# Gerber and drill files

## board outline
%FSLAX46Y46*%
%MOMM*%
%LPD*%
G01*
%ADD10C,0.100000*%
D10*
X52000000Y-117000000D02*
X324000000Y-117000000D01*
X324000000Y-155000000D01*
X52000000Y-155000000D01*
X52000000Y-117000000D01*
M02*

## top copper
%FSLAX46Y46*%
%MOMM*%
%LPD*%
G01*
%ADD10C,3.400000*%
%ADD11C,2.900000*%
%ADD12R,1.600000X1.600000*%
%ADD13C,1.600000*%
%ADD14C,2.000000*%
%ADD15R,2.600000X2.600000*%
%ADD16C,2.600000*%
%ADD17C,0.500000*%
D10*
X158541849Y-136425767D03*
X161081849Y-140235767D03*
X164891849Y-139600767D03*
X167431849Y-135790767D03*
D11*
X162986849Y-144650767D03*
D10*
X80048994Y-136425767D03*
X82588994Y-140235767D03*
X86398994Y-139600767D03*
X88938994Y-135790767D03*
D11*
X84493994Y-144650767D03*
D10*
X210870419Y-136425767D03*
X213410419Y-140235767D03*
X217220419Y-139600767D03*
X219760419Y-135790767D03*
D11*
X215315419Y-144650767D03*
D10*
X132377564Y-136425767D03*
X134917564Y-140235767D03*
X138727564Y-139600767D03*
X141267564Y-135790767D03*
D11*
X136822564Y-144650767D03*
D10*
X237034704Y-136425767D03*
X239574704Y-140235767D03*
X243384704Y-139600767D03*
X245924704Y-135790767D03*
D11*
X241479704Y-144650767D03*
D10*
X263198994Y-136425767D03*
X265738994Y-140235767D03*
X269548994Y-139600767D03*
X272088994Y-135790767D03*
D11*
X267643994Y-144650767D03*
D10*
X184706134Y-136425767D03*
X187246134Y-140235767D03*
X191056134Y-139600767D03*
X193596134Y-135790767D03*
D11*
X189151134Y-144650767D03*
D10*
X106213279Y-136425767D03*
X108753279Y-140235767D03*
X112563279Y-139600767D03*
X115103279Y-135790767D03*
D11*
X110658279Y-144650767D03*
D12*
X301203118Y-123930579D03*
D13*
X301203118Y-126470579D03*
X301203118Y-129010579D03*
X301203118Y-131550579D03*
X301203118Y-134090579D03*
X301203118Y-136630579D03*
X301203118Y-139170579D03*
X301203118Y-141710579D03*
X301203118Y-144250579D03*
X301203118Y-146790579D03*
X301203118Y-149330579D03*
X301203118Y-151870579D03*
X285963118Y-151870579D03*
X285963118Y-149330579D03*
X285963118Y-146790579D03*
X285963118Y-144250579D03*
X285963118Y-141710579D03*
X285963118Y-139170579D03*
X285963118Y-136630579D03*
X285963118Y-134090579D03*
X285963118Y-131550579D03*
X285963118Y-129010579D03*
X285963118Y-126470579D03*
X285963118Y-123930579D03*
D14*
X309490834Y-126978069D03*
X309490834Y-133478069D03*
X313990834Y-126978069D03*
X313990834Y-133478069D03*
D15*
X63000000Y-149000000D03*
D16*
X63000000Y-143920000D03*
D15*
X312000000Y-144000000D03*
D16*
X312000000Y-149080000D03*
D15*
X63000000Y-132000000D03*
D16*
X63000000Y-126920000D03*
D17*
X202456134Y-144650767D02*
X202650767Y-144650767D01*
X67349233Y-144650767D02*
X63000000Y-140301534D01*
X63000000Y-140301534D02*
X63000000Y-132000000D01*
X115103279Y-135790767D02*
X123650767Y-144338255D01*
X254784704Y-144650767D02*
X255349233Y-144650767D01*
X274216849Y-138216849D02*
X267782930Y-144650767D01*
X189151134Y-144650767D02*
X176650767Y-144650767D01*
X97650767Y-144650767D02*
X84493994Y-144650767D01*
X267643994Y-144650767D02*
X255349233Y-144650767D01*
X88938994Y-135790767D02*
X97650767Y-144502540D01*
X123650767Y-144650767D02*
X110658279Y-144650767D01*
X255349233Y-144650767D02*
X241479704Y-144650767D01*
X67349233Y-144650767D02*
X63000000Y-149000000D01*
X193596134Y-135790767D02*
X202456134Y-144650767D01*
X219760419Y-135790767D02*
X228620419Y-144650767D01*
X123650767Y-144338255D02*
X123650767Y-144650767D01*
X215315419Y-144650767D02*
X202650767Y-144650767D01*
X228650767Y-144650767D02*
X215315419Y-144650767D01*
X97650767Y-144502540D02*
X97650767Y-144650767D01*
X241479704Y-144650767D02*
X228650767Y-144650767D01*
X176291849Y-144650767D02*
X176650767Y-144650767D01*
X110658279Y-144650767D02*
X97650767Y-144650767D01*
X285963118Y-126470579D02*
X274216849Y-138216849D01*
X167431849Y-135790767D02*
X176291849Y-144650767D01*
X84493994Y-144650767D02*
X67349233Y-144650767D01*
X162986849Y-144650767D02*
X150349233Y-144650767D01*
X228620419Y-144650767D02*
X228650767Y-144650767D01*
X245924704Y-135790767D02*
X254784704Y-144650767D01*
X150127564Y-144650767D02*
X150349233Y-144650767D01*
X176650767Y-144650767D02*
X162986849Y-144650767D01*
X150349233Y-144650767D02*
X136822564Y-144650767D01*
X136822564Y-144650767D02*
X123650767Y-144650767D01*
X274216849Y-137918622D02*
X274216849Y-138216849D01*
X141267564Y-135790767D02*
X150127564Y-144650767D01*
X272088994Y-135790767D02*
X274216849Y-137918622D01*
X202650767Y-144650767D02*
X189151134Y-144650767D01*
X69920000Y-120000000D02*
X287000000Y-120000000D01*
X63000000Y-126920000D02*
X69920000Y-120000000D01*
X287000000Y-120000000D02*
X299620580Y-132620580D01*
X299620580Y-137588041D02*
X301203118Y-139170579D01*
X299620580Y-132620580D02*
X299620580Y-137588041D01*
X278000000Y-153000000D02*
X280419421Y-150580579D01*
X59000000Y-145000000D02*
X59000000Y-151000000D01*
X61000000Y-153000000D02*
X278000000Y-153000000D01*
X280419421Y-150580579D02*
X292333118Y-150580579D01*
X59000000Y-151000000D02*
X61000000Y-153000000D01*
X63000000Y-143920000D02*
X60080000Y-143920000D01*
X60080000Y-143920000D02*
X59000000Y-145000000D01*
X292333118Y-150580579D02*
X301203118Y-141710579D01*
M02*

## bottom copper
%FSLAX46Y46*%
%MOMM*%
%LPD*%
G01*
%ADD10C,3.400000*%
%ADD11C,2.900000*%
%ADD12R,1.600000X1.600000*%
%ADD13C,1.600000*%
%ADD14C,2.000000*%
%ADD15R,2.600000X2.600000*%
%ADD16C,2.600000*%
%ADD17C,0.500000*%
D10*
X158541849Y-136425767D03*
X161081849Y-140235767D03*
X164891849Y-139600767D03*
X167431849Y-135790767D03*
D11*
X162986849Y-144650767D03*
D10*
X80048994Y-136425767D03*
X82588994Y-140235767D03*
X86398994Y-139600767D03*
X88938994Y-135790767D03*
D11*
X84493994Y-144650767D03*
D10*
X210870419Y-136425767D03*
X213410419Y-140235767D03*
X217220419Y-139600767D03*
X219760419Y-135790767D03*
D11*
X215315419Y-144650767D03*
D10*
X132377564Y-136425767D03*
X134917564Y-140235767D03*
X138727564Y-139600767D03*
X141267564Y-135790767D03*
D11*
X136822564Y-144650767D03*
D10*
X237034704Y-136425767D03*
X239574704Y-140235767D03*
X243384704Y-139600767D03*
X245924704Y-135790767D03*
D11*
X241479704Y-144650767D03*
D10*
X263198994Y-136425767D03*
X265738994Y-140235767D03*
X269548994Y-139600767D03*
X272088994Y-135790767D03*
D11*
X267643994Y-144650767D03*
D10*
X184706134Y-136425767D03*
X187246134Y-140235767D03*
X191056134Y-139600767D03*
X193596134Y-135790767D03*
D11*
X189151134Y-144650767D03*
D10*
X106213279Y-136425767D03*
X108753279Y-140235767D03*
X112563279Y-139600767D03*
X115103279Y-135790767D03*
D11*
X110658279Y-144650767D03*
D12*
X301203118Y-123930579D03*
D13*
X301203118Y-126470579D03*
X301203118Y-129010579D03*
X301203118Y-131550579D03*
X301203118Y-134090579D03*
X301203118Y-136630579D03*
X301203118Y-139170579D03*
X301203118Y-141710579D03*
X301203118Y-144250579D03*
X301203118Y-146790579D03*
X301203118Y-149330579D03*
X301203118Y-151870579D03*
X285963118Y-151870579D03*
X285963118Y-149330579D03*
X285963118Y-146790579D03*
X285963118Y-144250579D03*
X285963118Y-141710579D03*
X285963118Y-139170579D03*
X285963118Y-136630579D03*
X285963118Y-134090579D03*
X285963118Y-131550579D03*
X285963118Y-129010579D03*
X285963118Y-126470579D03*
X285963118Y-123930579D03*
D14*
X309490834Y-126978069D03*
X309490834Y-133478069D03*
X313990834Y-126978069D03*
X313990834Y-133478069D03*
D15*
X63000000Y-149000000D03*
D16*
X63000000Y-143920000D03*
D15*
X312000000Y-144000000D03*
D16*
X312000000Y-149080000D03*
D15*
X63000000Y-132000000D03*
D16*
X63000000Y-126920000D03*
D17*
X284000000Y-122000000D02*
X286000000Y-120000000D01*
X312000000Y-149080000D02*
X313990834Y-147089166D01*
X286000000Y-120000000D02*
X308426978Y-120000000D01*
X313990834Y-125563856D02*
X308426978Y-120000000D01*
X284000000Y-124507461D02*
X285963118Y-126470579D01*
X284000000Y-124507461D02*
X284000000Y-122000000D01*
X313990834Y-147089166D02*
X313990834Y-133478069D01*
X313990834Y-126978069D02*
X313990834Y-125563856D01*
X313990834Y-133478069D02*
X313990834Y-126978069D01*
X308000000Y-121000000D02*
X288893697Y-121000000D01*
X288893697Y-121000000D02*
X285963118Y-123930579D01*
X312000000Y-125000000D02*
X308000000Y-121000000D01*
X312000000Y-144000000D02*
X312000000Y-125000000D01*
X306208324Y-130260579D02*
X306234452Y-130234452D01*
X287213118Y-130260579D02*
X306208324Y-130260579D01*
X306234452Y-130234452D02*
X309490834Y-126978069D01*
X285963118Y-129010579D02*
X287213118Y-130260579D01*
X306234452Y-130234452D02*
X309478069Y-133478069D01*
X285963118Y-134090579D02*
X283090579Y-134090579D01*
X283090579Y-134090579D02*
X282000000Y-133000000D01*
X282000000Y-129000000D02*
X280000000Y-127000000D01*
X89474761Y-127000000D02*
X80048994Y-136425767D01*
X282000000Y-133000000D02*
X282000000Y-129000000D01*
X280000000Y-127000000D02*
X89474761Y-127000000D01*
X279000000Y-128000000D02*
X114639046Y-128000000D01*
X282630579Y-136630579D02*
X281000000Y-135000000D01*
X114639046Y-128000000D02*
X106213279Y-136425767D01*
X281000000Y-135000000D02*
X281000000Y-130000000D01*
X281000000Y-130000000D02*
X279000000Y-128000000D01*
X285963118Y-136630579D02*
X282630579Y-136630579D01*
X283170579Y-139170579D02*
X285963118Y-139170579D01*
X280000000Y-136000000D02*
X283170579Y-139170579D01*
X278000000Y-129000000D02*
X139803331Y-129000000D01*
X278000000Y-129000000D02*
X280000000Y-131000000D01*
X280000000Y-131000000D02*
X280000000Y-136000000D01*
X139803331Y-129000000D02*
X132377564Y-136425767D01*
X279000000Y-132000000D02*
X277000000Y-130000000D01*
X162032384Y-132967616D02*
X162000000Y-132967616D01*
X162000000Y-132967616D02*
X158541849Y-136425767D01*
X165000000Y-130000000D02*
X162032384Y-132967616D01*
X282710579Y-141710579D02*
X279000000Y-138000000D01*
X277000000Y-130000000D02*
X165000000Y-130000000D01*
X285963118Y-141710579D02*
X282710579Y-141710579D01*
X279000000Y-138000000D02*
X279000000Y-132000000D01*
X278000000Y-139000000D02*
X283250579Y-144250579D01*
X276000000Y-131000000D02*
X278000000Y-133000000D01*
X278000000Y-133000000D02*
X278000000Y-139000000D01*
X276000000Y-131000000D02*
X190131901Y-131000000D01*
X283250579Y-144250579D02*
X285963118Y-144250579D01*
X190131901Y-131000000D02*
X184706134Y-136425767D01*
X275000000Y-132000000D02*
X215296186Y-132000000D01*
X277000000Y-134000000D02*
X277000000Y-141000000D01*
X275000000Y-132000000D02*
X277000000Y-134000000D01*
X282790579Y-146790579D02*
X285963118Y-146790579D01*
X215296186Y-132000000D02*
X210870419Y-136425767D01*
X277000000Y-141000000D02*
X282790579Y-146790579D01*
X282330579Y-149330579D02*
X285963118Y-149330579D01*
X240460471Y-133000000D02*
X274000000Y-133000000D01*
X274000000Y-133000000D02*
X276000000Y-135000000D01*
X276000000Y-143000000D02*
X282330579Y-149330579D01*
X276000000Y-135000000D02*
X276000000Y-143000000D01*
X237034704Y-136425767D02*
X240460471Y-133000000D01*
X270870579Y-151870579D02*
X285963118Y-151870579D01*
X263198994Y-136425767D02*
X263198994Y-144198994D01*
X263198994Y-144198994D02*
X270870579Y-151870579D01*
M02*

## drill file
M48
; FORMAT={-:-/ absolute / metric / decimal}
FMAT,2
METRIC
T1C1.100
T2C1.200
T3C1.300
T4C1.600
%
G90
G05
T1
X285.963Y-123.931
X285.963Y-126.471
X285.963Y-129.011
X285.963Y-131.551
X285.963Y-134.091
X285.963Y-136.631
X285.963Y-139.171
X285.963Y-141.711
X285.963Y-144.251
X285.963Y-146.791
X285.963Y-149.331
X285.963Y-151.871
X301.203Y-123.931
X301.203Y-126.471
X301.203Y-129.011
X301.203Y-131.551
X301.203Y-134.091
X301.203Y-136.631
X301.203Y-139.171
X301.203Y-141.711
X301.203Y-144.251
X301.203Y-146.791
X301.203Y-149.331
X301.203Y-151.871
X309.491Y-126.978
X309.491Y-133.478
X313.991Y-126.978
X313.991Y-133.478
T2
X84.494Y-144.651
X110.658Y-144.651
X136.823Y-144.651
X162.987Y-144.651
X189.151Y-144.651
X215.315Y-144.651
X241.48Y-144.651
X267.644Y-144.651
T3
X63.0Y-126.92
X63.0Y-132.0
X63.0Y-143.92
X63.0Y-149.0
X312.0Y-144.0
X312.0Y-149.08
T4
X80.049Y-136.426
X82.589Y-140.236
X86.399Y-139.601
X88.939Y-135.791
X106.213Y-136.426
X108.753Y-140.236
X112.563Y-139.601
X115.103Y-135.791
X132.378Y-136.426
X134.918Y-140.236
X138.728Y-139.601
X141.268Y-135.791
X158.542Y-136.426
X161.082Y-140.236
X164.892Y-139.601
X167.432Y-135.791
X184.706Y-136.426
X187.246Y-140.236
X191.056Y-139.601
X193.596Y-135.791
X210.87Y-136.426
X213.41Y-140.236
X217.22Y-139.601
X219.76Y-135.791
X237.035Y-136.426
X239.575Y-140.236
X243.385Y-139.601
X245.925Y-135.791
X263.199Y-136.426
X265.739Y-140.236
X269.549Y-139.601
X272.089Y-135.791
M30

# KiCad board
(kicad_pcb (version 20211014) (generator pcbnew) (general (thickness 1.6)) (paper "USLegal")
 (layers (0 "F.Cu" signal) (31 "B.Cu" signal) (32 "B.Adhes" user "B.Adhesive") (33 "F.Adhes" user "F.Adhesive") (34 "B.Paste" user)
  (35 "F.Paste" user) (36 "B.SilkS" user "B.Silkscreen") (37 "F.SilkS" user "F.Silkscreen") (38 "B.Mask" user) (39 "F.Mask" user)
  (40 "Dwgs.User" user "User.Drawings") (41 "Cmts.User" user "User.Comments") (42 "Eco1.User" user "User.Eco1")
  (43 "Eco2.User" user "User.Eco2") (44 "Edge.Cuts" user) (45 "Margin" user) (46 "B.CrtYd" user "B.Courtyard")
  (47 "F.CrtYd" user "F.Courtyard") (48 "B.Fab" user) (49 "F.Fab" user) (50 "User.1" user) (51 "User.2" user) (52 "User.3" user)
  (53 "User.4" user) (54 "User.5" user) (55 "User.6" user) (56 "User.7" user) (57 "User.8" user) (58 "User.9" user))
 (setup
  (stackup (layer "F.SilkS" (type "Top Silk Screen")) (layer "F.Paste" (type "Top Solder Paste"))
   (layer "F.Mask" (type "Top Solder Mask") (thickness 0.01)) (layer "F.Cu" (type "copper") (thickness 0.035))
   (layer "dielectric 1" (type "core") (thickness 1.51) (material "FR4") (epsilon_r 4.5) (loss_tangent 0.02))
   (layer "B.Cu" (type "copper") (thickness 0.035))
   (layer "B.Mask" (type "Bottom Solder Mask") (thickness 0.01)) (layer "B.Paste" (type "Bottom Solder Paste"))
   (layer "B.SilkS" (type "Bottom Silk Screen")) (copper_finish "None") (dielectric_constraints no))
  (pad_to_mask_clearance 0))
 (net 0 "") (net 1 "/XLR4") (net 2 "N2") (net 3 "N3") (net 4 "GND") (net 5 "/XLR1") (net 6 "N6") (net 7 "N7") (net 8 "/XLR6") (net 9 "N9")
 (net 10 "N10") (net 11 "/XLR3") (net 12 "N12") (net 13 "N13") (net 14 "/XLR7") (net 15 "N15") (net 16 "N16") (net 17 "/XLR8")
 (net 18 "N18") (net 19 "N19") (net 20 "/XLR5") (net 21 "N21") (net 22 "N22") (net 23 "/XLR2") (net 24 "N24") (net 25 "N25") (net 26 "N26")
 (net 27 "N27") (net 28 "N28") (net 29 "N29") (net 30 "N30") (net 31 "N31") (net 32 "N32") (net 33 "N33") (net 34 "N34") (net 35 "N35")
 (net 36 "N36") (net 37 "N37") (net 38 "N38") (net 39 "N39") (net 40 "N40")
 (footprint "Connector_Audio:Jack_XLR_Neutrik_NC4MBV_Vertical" (layer "F.Cu") (at 158.541849 136.425767)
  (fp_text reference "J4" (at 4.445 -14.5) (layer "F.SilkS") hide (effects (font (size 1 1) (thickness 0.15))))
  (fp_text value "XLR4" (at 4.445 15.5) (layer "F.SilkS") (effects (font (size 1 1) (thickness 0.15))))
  (pad "1" thru_hole circle (at 0 0) (size 3.4 3.4) (drill 1.6) (layers *.Cu *.Mask) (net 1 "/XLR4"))
  (pad "2" thru_hole circle (at 2.54 3.81) (size 3.4 3.4) (drill 1.6) (layers *.Cu *.Mask) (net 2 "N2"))
  (pad "3" thru_hole circle (at 6.35 3.175) (size 3.4 3.4) (drill 1.6) (layers *.Cu *.Mask) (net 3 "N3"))
  (pad "4" thru_hole circle (at 8.89 -0.635) (size 3.4 3.4) (drill 1.6) (layers *.Cu *.Mask) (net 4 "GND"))
  (pad "G" thru_hole circle (at 4.445 8.225) (size 2.9 2.9) (drill 1.2) (layers *.Cu *.Mask) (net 4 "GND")))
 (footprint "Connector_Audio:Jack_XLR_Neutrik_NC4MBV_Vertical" (layer "F.Cu") (at 80.048994 136.425767)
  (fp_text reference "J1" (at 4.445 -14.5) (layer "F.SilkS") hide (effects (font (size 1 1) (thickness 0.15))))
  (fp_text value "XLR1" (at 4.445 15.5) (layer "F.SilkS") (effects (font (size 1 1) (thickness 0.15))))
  (pad "1" thru_hole circle (at 0 0) (size 3.4 3.4) (drill 1.6) (layers *.Cu *.Mask) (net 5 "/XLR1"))
  (pad "2" thru_hole circle (at 2.54 3.81) (size 3.4 3.4) (drill 1.6) (layers *.Cu *.Mask) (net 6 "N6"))
  (pad "3" thru_hole circle (at 6.35 3.175) (size 3.4 3.4) (drill 1.6) (layers *.Cu *.Mask) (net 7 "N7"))
  (pad "4" thru_hole circle (at 8.89 -0.635) (size 3.4 3.4) (drill 1.6) (layers *.Cu *.Mask) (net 4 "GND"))
  (pad "G" thru_hole circle (at 4.445 8.225) (size 2.9 2.9) (drill 1.2) (layers *.Cu *.Mask) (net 4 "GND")))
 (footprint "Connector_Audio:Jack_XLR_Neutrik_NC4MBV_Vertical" (layer "F.Cu") (at 210.870419 136.425767)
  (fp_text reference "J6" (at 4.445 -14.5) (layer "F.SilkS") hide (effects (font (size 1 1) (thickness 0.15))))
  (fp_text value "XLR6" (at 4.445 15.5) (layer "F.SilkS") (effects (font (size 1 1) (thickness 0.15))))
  (pad "1" thru_hole circle (at 0 0) (size 3.4 3.4) (drill 1.6) (layers *.Cu *.Mask) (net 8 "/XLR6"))
  (pad "2" thru_hole circle (at 2.54 3.81) (size 3.4 3.4) (drill 1.6) (layers *.Cu *.Mask) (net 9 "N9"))
  (pad "3" thru_hole circle (at 6.35 3.175) (size 3.4 3.4) (drill 1.6) (layers *.Cu *.Mask) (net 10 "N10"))
  (pad "4" thru_hole circle (at 8.89 -0.635) (size 3.4 3.4) (drill 1.6) (layers *.Cu *.Mask) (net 4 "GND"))
  (pad "G" thru_hole circle (at 4.445 8.225) (size 2.9 2.9) (drill 1.2) (layers *.Cu *.Mask) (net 4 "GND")))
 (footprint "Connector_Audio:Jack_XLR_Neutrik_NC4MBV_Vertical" (layer "F.Cu") (at 132.377564 136.425767)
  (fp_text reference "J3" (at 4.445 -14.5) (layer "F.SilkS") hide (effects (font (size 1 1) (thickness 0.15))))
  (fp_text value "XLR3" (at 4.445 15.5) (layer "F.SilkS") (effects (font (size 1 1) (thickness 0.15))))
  (pad "1" thru_hole circle (at 0 0) (size 3.4 3.4) (drill 1.6) (layers *.Cu *.Mask) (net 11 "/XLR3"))
  (pad "2" thru_hole circle (at 2.54 3.81) (size 3.4 3.4) (drill 1.6) (layers *.Cu *.Mask) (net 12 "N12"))
  (pad "3" thru_hole circle (at 6.35 3.175) (size 3.4 3.4) (drill 1.6) (layers *.Cu *.Mask) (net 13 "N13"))
  (pad "4" thru_hole circle (at 8.89 -0.635) (size 3.4 3.4) (drill 1.6) (layers *.Cu *.Mask) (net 4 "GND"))
  (pad "G" thru_hole circle (at 4.445 8.225) (size 2.9 2.9) (drill 1.2) (layers *.Cu *.Mask) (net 4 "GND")))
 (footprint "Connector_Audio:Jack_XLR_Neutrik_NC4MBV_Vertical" (layer "F.Cu") (at 237.034704 136.425767)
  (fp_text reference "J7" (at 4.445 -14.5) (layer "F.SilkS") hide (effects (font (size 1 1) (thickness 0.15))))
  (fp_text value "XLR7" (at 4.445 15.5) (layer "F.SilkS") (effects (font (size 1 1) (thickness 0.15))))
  (pad "1" thru_hole circle (at 0 0) (size 3.4 3.4) (drill 1.6) (layers *.Cu *.Mask) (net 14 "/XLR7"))
  (pad "2" thru_hole circle (at 2.54 3.81) (size 3.4 3.4) (drill 1.6) (layers *.Cu *.Mask) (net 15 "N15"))
  (pad "3" thru_hole circle (at 6.35 3.175) (size 3.4 3.4) (drill 1.6) (layers *.Cu *.Mask) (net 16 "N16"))
  (pad "4" thru_hole circle (at 8.89 -0.635) (size 3.4 3.4) (drill 1.6) (layers *.Cu *.Mask) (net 4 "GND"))
  (pad "G" thru_hole circle (at 4.445 8.225) (size 2.9 2.9) (drill 1.2) (layers *.Cu *.Mask) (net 4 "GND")))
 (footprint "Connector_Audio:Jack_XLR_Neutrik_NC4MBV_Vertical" (layer "F.Cu") (at 263.198994 136.425767)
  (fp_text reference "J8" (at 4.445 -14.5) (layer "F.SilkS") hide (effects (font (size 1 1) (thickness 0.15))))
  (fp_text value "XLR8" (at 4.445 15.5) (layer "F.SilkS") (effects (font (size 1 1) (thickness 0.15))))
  (pad "1" thru_hole circle (at 0 0) (size 3.4 3.4) (drill 1.6) (layers *.Cu *.Mask) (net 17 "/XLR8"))
  (pad "2" thru_hole circle (at 2.54 3.81) (size 3.4 3.4) (drill 1.6) (layers *.Cu *.Mask) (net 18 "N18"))
  (pad "3" thru_hole circle (at 6.35 3.175) (size 3.4 3.4) (drill 1.6) (layers *.Cu *.Mask) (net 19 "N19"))
  (pad "4" thru_hole circle (at 8.89 -0.635) (size 3.4 3.4) (drill 1.6) (layers *.Cu *.Mask) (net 4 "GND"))
  (pad "G" thru_hole circle (at 4.445 8.225) (size 2.9 2.9) (drill 1.2) (layers *.Cu *.Mask) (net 4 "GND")))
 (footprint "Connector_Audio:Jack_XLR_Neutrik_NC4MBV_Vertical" (layer "F.Cu") (at 184.706134 136.425767)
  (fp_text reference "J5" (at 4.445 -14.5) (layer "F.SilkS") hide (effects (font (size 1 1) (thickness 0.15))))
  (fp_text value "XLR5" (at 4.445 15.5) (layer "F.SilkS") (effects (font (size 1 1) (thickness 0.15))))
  (pad "1" thru_hole circle (at 0 0) (size 3.4 3.4) (drill 1.6) (layers *.Cu *.Mask) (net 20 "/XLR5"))
  (pad "2" thru_hole circle (at 2.54 3.81) (size 3.4 3.4) (drill 1.6) (layers *.Cu *.Mask) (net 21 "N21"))
  (pad "3" thru_hole circle (at 6.35 3.175) (size 3.4 3.4) (drill 1.6) (layers *.Cu *.Mask) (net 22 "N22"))
  (pad "4" thru_hole circle (at 8.89 -0.635) (size 3.4 3.4) (drill 1.6) (layers *.Cu *.Mask) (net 4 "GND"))
  (pad "G" thru_hole circle (at 4.445 8.225) (size 2.9 2.9) (drill 1.2) (layers *.Cu *.Mask) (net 4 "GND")))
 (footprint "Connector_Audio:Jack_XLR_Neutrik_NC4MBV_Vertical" (layer "F.Cu") (at 106.213279 136.425767)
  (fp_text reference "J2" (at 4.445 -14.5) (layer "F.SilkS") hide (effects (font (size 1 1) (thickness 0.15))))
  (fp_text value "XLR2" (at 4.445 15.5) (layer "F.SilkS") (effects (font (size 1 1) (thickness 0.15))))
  (pad "1" thru_hole circle (at 0 0) (size 3.4 3.4) (drill 1.6) (layers *.Cu *.Mask) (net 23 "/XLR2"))
  (pad "2" thru_hole circle (at 2.54 3.81) (size 3.4 3.4) (drill 1.6) (layers *.Cu *.Mask) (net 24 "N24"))
  (pad "3" thru_hole circle (at 6.35 3.175) (size 3.4 3.4) (drill 1.6) (layers *.Cu *.Mask) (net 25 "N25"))
  (pad "4" thru_hole circle (at 8.89 -0.635) (size 3.4 3.4) (drill 1.6) (layers *.Cu *.Mask) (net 4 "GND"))
  (pad "G" thru_hole circle (at 4.445 8.225) (size 2.9 2.9) (drill 1.2) (layers *.Cu *.Mask) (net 4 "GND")))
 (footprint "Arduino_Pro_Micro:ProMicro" (layer "B.Cu") (at 293.583118 137.900579 -90)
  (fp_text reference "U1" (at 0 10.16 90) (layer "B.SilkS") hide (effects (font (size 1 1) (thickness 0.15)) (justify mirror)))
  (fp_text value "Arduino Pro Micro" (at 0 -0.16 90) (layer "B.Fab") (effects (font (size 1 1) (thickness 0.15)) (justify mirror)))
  (pad "1" thru_hole rect locked (at -13.97 -7.62 270) (size 1.6 1.6) (drill 1.1) (layers *.Cu *.Mask "B.SilkS") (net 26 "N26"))
  (pad "2" thru_hole circle locked (at -11.43 -7.62 270) (size 1.6 1.6) (drill 1.1) (layers *.Cu *.Mask "B.SilkS") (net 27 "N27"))
  (pad "3" thru_hole circle locked (at -8.89 -7.62 270) (size 1.6 1.6) (drill 1.1) (layers *.Cu *.Mask "B.SilkS") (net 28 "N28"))
  (pad "4" thru_hole circle locked (at -6.35 -7.62 270) (size 1.6 1.6) (drill 1.1) (layers *.Cu *.Mask "B.SilkS") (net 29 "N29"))
  (pad "5" thru_hole circle locked (at -3.81 -7.62 270) (size 1.6 1.6) (drill 1.1) (layers *.Cu *.Mask "B.SilkS") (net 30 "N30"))
  (pad "6" thru_hole circle locked (at -1.27 -7.62 270) (size 1.6 1.6) (drill 1.1) (layers *.Cu *.Mask "B.SilkS") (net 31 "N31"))
  (pad "7" thru_hole circle locked (at 1.27 -7.62 270) (size 1.6 1.6) (drill 1.1) (layers *.Cu *.Mask "B.SilkS") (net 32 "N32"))
  (pad "8" thru_hole circle locked (at 3.81 -7.62 270) (size 1.6 1.6) (drill 1.1) (layers *.Cu *.Mask "B.SilkS") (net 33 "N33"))
  (pad "9" thru_hole circle locked (at 6.35 -7.62 270) (size 1.6 1.6) (drill 1.1) (layers *.Cu *.Mask "B.SilkS") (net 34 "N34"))
  (pad "10" thru_hole circle locked (at 8.89 -7.62 270) (size 1.6 1.6) (drill 1.1) (layers *.Cu *.Mask "B.SilkS") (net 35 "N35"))
  (pad "11" thru_hole circle locked (at 11.43 -7.62 270) (size 1.6 1.6) (drill 1.1) (layers *.Cu *.Mask "B.SilkS") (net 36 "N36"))
  (pad "12" thru_hole circle locked (at 13.97 -7.62 270) (size 1.6 1.6) (drill 1.1) (layers *.Cu *.Mask "B.SilkS") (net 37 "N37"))
  (pad "13" thru_hole circle locked (at 13.97 7.62 270) (size 1.6 1.6) (drill 1.1) (layers *.Cu *.Mask "B.SilkS") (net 17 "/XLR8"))
  (pad "14" thru_hole circle locked (at 11.43 7.62 270) (size 1.6 1.6) (drill 1.1) (layers *.Cu *.Mask "B.SilkS") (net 14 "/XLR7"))
  (pad "15" thru_hole circle locked (at 8.89 7.62 270) (size 1.6 1.6) (drill 1.1) (layers *.Cu *.Mask "B.SilkS") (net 8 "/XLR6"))
  (pad "16" thru_hole circle locked (at 6.35 7.62 270) (size 1.6 1.6) (drill 1.1) (layers *.Cu *.Mask "B.SilkS") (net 20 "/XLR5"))
  (pad "17" thru_hole circle locked (at 3.81 7.62 270) (size 1.6 1.6) (drill 1.1) (layers *.Cu *.Mask "B.SilkS") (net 1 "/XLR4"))
  (pad "18" thru_hole circle locked (at 1.27 7.62 270) (size 1.6 1.6) (drill 1.1) (layers *.Cu *.Mask "B.SilkS") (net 11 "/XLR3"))
  (pad "19" thru_hole circle locked (at -1.27 7.62 270) (size 1.6 1.6) (drill 1.1) (layers *.Cu *.Mask "B.SilkS") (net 23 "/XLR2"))
  (pad "20" thru_hole circle locked (at -3.81 7.62 270) (size 1.6 1.6) (drill 1.1) (layers *.Cu *.Mask "B.SilkS") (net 5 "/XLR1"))
  (pad "21" thru_hole circle locked (at -6.35 7.62 270) (size 1.6 1.6) (drill 1.1) (layers *.Cu *.Mask "B.SilkS") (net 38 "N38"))
  (pad "22" thru_hole circle locked (at -8.89 7.62 270) (size 1.6 1.6) (drill 1.1) (layers *.Cu *.Mask "B.SilkS") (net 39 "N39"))
  (pad "23" thru_hole circle locked (at -11.43 7.62 270) (size 1.6 1.6) (drill 1.1) (layers *.Cu *.Mask "B.SilkS") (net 4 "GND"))
  (pad "24" thru_hole circle locked (at -13.97 7.62 270) (size 1.6 1.6) (drill 1.1) (layers *.Cu *.Mask "B.SilkS") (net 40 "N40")))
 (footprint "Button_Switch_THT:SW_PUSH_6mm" (layer "B.Cu") (at 309.490834 126.978069 -90)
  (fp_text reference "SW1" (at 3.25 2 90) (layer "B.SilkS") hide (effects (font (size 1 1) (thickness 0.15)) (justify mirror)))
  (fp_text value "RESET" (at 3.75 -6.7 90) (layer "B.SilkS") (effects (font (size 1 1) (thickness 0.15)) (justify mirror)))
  (pad "1" thru_hole circle (at 0 0 180) (size 2 2) (drill 1.1) (layers *.Cu *.Mask) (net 39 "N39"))
  (pad "1" thru_hole circle (at 6.5 0 180) (size 2 2) (drill 1.1) (layers *.Cu *.Mask) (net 39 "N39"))
  (pad "2" thru_hole circle (at 0 -4.5 180) (size 2 2) (drill 1.1) (layers *.Cu *.Mask) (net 4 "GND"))
  (pad "2" thru_hole circle (at 6.5 -4.5 180) (size 2 2) (drill 1.1) (layers *.Cu *.Mask) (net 4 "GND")))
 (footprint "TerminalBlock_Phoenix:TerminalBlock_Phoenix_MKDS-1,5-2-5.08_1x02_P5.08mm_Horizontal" (layer "B.Cu") (at 63 149 90)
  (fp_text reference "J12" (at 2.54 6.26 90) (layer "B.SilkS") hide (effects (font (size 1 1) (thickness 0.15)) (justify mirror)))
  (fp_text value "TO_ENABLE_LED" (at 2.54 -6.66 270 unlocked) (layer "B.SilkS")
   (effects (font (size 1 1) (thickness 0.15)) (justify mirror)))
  (pad "1" thru_hole rect (at 0 0 90) (size 2.6 2.6) (drill 1.3) (layers *.Cu *.Mask) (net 4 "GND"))
  (pad "2" thru_hole circle (at 5.08 0 90) (size 2.6 2.6) (drill 1.3) (layers *.Cu *.Mask) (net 33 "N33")))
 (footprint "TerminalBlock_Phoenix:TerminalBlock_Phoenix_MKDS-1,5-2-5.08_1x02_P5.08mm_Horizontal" (layer "B.Cu") (at 312 144 -90)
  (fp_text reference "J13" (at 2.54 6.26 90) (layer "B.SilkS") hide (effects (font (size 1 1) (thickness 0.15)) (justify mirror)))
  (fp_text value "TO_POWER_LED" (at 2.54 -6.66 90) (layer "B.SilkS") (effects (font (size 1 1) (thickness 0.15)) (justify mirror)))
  (pad "1" thru_hole rect (at 0 0 270) (size 2.6 2.6) (drill 1.3) (layers *.Cu *.Mask) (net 40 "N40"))
  (pad "2" thru_hole circle (at 5.08 0 270) (size 2.6 2.6) (drill 1.3) (layers *.Cu *.Mask) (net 4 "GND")))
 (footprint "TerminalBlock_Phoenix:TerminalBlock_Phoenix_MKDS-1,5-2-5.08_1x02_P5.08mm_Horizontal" (layer "B.Cu") (at 63 132 90)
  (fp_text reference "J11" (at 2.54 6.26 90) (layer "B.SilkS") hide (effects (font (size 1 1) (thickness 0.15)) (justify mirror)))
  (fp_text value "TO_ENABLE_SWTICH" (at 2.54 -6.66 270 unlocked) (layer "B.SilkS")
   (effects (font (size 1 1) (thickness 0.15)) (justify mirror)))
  (pad "1" thru_hole rect (at 0 0 90) (size 2.6 2.6) (drill 1.3) (layers *.Cu *.Mask) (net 4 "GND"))
  (pad "2" thru_hole circle (at 5.08 0 90) (size 2.6 2.6) (drill 1.3) (layers *.Cu *.Mask) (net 32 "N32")))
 (gr_rect (start 52 117) (end 324 155) (layer "Edge.Cuts") (width 0.1) (fill none))
 (segment (start 202.456134 144.650767) (end 202.650767 144.650767) (width 0.5) (layer "F.Cu") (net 4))
 (segment (start 67.349233 144.650767) (end 63 140.301534) (width 0.5) (layer "F.Cu") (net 4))
 (segment (start 63 140.301534) (end 63 132) (width 0.5) (layer "F.Cu") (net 4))
 (segment (start 115.103279 135.790767) (end 123.650767 144.338255) (width 0.5) (layer "F.Cu") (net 4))
 (segment (start 254.784704 144.650767) (end 255.349233 144.650767) (width 0.5) (layer "F.Cu") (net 4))
 (segment (start 274.216849 138.216849) (end 267.78293 144.650767) (width 0.5) (layer "F.Cu") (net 4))
 (segment (start 189.151134 144.650767) (end 176.650767 144.650767) (width 0.5) (layer "F.Cu") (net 4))
 (segment (start 97.650767 144.650767) (end 84.493994 144.650767) (width 0.5) (layer "F.Cu") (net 4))
 (segment (start 267.643994 144.650767) (end 255.349233 144.650767) (width 0.5) (layer "F.Cu") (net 4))
 (segment (start 88.938994 135.790767) (end 97.650767 144.50254) (width 0.5) (layer "F.Cu") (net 4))
 (segment (start 123.650767 144.650767) (end 110.658279 144.650767) (width 0.5) (layer "F.Cu") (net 4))
 (segment (start 255.349233 144.650767) (end 241.479704 144.650767) (width 0.5) (layer "F.Cu") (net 4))
 (segment (start 67.349233 144.650767) (end 63 149) (width 0.5) (layer "F.Cu") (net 4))
 (segment (start 193.596134 135.790767) (end 202.456134 144.650767) (width 0.5) (layer "F.Cu") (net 4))
 (segment (start 219.760419 135.790767) (end 228.620419 144.650767) (width 0.5) (layer "F.Cu") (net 4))
 (segment (start 123.650767 144.338255) (end 123.650767 144.650767) (width 0.5) (layer "F.Cu") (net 4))
 (segment (start 215.315419 144.650767) (end 202.650767 144.650767) (width 0.5) (layer "F.Cu") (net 4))
 (segment (start 228.650767 144.650767) (end 215.315419 144.650767) (width 0.5) (layer "F.Cu") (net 4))
 (segment (start 97.650767 144.50254) (end 97.650767 144.650767) (width 0.5) (layer "F.Cu") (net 4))
 (segment (start 241.479704 144.650767) (end 228.650767 144.650767) (width 0.5) (layer "F.Cu") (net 4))
 (segment (start 176.291849 144.650767) (end 176.650767 144.650767) (width 0.5) (layer "F.Cu") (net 4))
 (segment (start 110.658279 144.650767) (end 97.650767 144.650767) (width 0.5) (layer "F.Cu") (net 4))
 (segment (start 285.963118 126.470579) (end 274.216849 138.216849) (width 0.5) (layer "F.Cu") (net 4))
 (segment (start 167.431849 135.790767) (end 176.291849 144.650767) (width 0.5) (layer "F.Cu") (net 4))
 (segment (start 84.493994 144.650767) (end 67.349233 144.650767) (width 0.5) (layer "F.Cu") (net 4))
 (segment (start 162.986849 144.650767) (end 150.349233 144.650767) (width 0.5) (layer "F.Cu") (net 4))
 (segment (start 228.620419 144.650767) (end 228.650767 144.650767) (width 0.5) (layer "F.Cu") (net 4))
 (segment (start 245.924704 135.790767) (end 254.784704 144.650767) (width 0.5) (layer "F.Cu") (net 4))
 (segment (start 150.127564 144.650767) (end 150.349233 144.650767) (width 0.5) (layer "F.Cu") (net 4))
 (segment (start 176.650767 144.650767) (end 162.986849 144.650767) (width 0.5) (layer "F.Cu") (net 4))
 (segment (start 150.349233 144.650767) (end 136.822564 144.650767) (width 0.5) (layer "F.Cu") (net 4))
 (segment (start 136.822564 144.650767) (end 123.650767 144.650767) (width 0.5) (layer "F.Cu") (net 4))
 (segment (start 274.216849 137.918622) (end 274.216849 138.216849) (width 0.5) (layer "F.Cu") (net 4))
 (segment (start 141.267564 135.790767) (end 150.127564 144.650767) (width 0.5) (layer "F.Cu") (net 4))
 (segment (start 272.088994 135.790767) (end 274.216849 137.918622) (width 0.5) (layer "F.Cu") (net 4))
 (segment (start 202.650767 144.650767) (end 189.151134 144.650767) (width 0.5) (layer "F.Cu") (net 4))
 (segment (start 284 122) (end 286 120) (width 0.5) (layer "B.Cu") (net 4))
 (segment (start 312 149.08) (end 313.990834 147.089166) (width 0.5) (layer "B.Cu") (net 4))
 (segment (start 286 120) (end 308.426978 120) (width 0.5) (layer "B.Cu") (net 4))
 (segment (start 313.990834 125.563856) (end 308.426978 120) (width 0.5) (layer "B.Cu") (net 4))
 (segment (start 284 124.507461) (end 285.963118 126.470579) (width 0.5) (layer "B.Cu") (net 4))
 (segment (start 284 124.507461) (end 284 122) (width 0.5) (layer "B.Cu") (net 4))
 (segment (start 313.990834 147.089166) (end 313.990834 133.478069) (width 0.5) (layer "B.Cu") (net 4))
 (segment (start 313.990834 126.978069) (end 313.990834 125.563856) (width 0.5) (layer "B.Cu") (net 4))
 (segment (start 313.990834 133.478069) (end 313.990834 126.978069) (width 0.5) (layer "B.Cu") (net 4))
 (segment (start 69.92 120) (end 287 120) (width 0.5) (layer "F.Cu") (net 32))
 (segment (start 63 126.92) (end 69.92 120) (width 0.5) (layer "F.Cu") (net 32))
 (segment (start 287 120) (end 299.62058 132.62058) (width 0.5) (layer "F.Cu") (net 32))
 (segment (start 299.62058 137.588041) (end 301.203118 139.170579) (width 0.5) (layer "F.Cu") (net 32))
 (segment (start 299.62058 132.62058) (end 299.62058 137.588041) (width 0.5) (layer "F.Cu") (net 32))
 (segment (start 278 153) (end 280.419421 150.580579) (width 0.5) (layer "F.Cu") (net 33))
 (segment (start 59 145) (end 59 151) (width 0.5) (layer "F.Cu") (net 33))
 (segment (start 61 153) (end 278 153) (width 0.5) (layer "F.Cu") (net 33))
 (segment (start 280.419421 150.580579) (end 292.333118 150.580579) (width 0.5) (layer "F.Cu") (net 33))
 (segment (start 59 151) (end 61 153) (width 0.5) (layer "F.Cu") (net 33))
 (segment (start 63 143.92) (end 60.08 143.92) (width 0.5) (layer "F.Cu") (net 33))
 (segment (start 60.08 143.92) (end 59 145) (width 0.5) (layer "F.Cu") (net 33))
 (segment (start 292.333118 150.580579) (end 301.203118 141.710579) (width 0.5) (layer "F.Cu") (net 33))
 (segment (start 308 121) (end 288.893697 121) (width 0.5) (layer "B.Cu") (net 40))
 (segment (start 288.893697 121) (end 285.963118 123.930579) (width 0.5) (layer "B.Cu") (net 40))
 (segment (start 312 125) (end 308 121) (width 0.5) (layer "B.Cu") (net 40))
 (segment (start 312 144) (end 312 125) (width 0.5) (layer "B.Cu") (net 40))
 (segment (start 306.208324 130.260579) (end 306.234452 130.234452) (width 0.5) (layer "B.Cu") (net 39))
 (segment (start 287.213118 130.260579) (end 306.208324 130.260579) (width 0.5) (layer "B.Cu") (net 39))
 (segment (start 306.234452 130.234452) (end 309.490834 126.978069) (width 0.5) (layer "B.Cu") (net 39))
 (segment (start 285.963118 129.010579) (end 287.213118 130.260579) (width 0.5) (layer "B.Cu") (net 39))
 (segment (start 306.234452 130.234452) (end 309.478069 133.478069) (width 0.5) (layer "B.Cu") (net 39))
 (segment (start 285.963118 134.090579) (end 283.090579 134.090579) (width 0.5) (layer "B.Cu") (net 5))
 (segment (start 283.090579 134.090579) (end 282 133) (width 0.5) (layer "B.Cu") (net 5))
 (segment (start 282 129) (end 280 127) (width 0.5) (layer "B.Cu") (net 5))
 (segment (start 89.474761 127) (end 80.048994 136.425767) (width 0.5) (layer "B.Cu") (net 5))
 (segment (start 282 133) (end 282 129) (width 0.5) (layer "B.Cu") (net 5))
 (segment (start 280 127) (end 89.474761 127) (width 0.5) (layer "B.Cu") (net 5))
 (segment (start 279 128) (end 114.639046 128) (width 0.5) (layer "B.Cu") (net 23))
 (segment (start 282.630579 136.630579) (end 281 135) (width 0.5) (layer "B.Cu") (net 23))
 (segment (start 114.639046 128) (end 106.213279 136.425767) (width 0.5) (layer "B.Cu") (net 23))
 (segment (start 281 135) (end 281 130) (width 0.5) (layer "B.Cu") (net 23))
 (segment (start 281 130) (end 279 128) (width 0.5) (layer "B.Cu") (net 23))
 (segment (start 285.963118 136.630579) (end 282.630579 136.630579) (width 0.5) (layer "B.Cu") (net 23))
 (segment (start 283.170579 139.170579) (end 285.963118 139.170579) (width 0.5) (layer "B.Cu") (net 11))
 (segment (start 280 136) (end 283.170579 139.170579) (width 0.5) (layer "B.Cu") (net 11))
 (segment (start 278 129) (end 139.803331 129) (width 0.5) (layer "B.Cu") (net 11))
 (segment (start 278 129) (end 280 131) (width 0.5) (layer "B.Cu") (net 11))
 (segment (start 280 131) (end 280 136) (width 0.5) (layer "B.Cu") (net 11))
 (segment (start 139.803331 129) (end 132.377564 136.425767) (width 0.5) (layer "B.Cu") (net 11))
 (segment (start 279 132) (end 277 130) (width 0.5) (layer "B.Cu") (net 1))
 (segment (start 162.032384 132.967616) (end 162 132.967616) (width 0.5) (layer "B.Cu") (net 1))
 (segment (start 162 132.967616) (end 158.541849 136.425767) (width 0.5) (layer "B.Cu") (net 1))
 (segment (start 165 130) (end 162.032384 132.967616) (width 0.5) (layer "B.Cu") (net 1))
 (segment (start 282.710579 141.710579) (end 279 138) (width 0.5) (layer "B.Cu") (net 1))
 (segment (start 277 130) (end 165 130) (width 0.5) (layer "B.Cu") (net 1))
 (segment (start 285.963118 141.710579) (end 282.710579 141.710579) (width 0.5) (layer "B.Cu") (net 1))
 (segment (start 279 138) (end 279 132) (width 0.5) (layer "B.Cu") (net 1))
 (segment (start 278 139) (end 283.250579 144.250579) (width 0.5) (layer "B.Cu") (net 20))
 (segment (start 276 131) (end 278 133) (width 0.5) (layer "B.Cu") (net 20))
 (segment (start 278 133) (end 278 139) (width 0.5) (layer "B.Cu") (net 20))
 (segment (start 276 131) (end 190.131901 131) (width 0.5) (layer "B.Cu") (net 20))
 (segment (start 283.250579 144.250579) (end 285.963118 144.250579) (width 0.5) (layer "B.Cu") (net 20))
 (segment (start 190.131901 131) (end 184.706134 136.425767) (width 0.5) (layer "B.Cu") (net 20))
 (segment (start 275 132) (end 215.296186 132) (width 0.5) (layer "B.Cu") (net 8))
 (segment (start 277 134) (end 277 141) (width 0.5) (layer "B.Cu") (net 8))
 (segment (start 275 132) (end 277 134) (width 0.5) (layer "B.Cu") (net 8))
 (segment (start 282.790579 146.790579) (end 285.963118 146.790579) (width 0.5) (layer "B.Cu") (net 8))
 (segment (start 215.296186 132) (end 210.870419 136.425767) (width 0.5) (layer "B.Cu") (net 8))
 (segment (start 277 141) (end 282.790579 146.790579) (width 0.5) (layer "B.Cu") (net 8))
 (segment (start 282.330579 149.330579) (end 285.963118 149.330579) (width 0.5) (layer "B.Cu") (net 14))
 (segment (start 240.460471 133) (end 274 133) (width 0.5) (layer "B.Cu") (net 14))
 (segment (start 274 133) (end 276 135) (width 0.5) (layer "B.Cu") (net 14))
 (segment (start 276 143) (end 282.330579 149.330579) (width 0.5) (layer "B.Cu") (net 14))
 (segment (start 276 135) (end 276 143) (width 0.5) (layer "B.Cu") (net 14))
 (segment (start 237.034704 136.425767) (end 240.460471 133) (width 0.5) (layer "B.Cu") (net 14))
 (segment (start 270.870579 151.870579) (end 285.963118 151.870579) (width 0.5) (layer "B.Cu") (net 17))
 (segment (start 263.198994 136.425767) (end 263.198994 144.198994) (width 0.5) (layer "B.Cu") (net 17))
 (segment (start 263.198994 144.198994) (end 270.870579 151.870579) (width 0.5) (layer "B.Cu") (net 17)))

